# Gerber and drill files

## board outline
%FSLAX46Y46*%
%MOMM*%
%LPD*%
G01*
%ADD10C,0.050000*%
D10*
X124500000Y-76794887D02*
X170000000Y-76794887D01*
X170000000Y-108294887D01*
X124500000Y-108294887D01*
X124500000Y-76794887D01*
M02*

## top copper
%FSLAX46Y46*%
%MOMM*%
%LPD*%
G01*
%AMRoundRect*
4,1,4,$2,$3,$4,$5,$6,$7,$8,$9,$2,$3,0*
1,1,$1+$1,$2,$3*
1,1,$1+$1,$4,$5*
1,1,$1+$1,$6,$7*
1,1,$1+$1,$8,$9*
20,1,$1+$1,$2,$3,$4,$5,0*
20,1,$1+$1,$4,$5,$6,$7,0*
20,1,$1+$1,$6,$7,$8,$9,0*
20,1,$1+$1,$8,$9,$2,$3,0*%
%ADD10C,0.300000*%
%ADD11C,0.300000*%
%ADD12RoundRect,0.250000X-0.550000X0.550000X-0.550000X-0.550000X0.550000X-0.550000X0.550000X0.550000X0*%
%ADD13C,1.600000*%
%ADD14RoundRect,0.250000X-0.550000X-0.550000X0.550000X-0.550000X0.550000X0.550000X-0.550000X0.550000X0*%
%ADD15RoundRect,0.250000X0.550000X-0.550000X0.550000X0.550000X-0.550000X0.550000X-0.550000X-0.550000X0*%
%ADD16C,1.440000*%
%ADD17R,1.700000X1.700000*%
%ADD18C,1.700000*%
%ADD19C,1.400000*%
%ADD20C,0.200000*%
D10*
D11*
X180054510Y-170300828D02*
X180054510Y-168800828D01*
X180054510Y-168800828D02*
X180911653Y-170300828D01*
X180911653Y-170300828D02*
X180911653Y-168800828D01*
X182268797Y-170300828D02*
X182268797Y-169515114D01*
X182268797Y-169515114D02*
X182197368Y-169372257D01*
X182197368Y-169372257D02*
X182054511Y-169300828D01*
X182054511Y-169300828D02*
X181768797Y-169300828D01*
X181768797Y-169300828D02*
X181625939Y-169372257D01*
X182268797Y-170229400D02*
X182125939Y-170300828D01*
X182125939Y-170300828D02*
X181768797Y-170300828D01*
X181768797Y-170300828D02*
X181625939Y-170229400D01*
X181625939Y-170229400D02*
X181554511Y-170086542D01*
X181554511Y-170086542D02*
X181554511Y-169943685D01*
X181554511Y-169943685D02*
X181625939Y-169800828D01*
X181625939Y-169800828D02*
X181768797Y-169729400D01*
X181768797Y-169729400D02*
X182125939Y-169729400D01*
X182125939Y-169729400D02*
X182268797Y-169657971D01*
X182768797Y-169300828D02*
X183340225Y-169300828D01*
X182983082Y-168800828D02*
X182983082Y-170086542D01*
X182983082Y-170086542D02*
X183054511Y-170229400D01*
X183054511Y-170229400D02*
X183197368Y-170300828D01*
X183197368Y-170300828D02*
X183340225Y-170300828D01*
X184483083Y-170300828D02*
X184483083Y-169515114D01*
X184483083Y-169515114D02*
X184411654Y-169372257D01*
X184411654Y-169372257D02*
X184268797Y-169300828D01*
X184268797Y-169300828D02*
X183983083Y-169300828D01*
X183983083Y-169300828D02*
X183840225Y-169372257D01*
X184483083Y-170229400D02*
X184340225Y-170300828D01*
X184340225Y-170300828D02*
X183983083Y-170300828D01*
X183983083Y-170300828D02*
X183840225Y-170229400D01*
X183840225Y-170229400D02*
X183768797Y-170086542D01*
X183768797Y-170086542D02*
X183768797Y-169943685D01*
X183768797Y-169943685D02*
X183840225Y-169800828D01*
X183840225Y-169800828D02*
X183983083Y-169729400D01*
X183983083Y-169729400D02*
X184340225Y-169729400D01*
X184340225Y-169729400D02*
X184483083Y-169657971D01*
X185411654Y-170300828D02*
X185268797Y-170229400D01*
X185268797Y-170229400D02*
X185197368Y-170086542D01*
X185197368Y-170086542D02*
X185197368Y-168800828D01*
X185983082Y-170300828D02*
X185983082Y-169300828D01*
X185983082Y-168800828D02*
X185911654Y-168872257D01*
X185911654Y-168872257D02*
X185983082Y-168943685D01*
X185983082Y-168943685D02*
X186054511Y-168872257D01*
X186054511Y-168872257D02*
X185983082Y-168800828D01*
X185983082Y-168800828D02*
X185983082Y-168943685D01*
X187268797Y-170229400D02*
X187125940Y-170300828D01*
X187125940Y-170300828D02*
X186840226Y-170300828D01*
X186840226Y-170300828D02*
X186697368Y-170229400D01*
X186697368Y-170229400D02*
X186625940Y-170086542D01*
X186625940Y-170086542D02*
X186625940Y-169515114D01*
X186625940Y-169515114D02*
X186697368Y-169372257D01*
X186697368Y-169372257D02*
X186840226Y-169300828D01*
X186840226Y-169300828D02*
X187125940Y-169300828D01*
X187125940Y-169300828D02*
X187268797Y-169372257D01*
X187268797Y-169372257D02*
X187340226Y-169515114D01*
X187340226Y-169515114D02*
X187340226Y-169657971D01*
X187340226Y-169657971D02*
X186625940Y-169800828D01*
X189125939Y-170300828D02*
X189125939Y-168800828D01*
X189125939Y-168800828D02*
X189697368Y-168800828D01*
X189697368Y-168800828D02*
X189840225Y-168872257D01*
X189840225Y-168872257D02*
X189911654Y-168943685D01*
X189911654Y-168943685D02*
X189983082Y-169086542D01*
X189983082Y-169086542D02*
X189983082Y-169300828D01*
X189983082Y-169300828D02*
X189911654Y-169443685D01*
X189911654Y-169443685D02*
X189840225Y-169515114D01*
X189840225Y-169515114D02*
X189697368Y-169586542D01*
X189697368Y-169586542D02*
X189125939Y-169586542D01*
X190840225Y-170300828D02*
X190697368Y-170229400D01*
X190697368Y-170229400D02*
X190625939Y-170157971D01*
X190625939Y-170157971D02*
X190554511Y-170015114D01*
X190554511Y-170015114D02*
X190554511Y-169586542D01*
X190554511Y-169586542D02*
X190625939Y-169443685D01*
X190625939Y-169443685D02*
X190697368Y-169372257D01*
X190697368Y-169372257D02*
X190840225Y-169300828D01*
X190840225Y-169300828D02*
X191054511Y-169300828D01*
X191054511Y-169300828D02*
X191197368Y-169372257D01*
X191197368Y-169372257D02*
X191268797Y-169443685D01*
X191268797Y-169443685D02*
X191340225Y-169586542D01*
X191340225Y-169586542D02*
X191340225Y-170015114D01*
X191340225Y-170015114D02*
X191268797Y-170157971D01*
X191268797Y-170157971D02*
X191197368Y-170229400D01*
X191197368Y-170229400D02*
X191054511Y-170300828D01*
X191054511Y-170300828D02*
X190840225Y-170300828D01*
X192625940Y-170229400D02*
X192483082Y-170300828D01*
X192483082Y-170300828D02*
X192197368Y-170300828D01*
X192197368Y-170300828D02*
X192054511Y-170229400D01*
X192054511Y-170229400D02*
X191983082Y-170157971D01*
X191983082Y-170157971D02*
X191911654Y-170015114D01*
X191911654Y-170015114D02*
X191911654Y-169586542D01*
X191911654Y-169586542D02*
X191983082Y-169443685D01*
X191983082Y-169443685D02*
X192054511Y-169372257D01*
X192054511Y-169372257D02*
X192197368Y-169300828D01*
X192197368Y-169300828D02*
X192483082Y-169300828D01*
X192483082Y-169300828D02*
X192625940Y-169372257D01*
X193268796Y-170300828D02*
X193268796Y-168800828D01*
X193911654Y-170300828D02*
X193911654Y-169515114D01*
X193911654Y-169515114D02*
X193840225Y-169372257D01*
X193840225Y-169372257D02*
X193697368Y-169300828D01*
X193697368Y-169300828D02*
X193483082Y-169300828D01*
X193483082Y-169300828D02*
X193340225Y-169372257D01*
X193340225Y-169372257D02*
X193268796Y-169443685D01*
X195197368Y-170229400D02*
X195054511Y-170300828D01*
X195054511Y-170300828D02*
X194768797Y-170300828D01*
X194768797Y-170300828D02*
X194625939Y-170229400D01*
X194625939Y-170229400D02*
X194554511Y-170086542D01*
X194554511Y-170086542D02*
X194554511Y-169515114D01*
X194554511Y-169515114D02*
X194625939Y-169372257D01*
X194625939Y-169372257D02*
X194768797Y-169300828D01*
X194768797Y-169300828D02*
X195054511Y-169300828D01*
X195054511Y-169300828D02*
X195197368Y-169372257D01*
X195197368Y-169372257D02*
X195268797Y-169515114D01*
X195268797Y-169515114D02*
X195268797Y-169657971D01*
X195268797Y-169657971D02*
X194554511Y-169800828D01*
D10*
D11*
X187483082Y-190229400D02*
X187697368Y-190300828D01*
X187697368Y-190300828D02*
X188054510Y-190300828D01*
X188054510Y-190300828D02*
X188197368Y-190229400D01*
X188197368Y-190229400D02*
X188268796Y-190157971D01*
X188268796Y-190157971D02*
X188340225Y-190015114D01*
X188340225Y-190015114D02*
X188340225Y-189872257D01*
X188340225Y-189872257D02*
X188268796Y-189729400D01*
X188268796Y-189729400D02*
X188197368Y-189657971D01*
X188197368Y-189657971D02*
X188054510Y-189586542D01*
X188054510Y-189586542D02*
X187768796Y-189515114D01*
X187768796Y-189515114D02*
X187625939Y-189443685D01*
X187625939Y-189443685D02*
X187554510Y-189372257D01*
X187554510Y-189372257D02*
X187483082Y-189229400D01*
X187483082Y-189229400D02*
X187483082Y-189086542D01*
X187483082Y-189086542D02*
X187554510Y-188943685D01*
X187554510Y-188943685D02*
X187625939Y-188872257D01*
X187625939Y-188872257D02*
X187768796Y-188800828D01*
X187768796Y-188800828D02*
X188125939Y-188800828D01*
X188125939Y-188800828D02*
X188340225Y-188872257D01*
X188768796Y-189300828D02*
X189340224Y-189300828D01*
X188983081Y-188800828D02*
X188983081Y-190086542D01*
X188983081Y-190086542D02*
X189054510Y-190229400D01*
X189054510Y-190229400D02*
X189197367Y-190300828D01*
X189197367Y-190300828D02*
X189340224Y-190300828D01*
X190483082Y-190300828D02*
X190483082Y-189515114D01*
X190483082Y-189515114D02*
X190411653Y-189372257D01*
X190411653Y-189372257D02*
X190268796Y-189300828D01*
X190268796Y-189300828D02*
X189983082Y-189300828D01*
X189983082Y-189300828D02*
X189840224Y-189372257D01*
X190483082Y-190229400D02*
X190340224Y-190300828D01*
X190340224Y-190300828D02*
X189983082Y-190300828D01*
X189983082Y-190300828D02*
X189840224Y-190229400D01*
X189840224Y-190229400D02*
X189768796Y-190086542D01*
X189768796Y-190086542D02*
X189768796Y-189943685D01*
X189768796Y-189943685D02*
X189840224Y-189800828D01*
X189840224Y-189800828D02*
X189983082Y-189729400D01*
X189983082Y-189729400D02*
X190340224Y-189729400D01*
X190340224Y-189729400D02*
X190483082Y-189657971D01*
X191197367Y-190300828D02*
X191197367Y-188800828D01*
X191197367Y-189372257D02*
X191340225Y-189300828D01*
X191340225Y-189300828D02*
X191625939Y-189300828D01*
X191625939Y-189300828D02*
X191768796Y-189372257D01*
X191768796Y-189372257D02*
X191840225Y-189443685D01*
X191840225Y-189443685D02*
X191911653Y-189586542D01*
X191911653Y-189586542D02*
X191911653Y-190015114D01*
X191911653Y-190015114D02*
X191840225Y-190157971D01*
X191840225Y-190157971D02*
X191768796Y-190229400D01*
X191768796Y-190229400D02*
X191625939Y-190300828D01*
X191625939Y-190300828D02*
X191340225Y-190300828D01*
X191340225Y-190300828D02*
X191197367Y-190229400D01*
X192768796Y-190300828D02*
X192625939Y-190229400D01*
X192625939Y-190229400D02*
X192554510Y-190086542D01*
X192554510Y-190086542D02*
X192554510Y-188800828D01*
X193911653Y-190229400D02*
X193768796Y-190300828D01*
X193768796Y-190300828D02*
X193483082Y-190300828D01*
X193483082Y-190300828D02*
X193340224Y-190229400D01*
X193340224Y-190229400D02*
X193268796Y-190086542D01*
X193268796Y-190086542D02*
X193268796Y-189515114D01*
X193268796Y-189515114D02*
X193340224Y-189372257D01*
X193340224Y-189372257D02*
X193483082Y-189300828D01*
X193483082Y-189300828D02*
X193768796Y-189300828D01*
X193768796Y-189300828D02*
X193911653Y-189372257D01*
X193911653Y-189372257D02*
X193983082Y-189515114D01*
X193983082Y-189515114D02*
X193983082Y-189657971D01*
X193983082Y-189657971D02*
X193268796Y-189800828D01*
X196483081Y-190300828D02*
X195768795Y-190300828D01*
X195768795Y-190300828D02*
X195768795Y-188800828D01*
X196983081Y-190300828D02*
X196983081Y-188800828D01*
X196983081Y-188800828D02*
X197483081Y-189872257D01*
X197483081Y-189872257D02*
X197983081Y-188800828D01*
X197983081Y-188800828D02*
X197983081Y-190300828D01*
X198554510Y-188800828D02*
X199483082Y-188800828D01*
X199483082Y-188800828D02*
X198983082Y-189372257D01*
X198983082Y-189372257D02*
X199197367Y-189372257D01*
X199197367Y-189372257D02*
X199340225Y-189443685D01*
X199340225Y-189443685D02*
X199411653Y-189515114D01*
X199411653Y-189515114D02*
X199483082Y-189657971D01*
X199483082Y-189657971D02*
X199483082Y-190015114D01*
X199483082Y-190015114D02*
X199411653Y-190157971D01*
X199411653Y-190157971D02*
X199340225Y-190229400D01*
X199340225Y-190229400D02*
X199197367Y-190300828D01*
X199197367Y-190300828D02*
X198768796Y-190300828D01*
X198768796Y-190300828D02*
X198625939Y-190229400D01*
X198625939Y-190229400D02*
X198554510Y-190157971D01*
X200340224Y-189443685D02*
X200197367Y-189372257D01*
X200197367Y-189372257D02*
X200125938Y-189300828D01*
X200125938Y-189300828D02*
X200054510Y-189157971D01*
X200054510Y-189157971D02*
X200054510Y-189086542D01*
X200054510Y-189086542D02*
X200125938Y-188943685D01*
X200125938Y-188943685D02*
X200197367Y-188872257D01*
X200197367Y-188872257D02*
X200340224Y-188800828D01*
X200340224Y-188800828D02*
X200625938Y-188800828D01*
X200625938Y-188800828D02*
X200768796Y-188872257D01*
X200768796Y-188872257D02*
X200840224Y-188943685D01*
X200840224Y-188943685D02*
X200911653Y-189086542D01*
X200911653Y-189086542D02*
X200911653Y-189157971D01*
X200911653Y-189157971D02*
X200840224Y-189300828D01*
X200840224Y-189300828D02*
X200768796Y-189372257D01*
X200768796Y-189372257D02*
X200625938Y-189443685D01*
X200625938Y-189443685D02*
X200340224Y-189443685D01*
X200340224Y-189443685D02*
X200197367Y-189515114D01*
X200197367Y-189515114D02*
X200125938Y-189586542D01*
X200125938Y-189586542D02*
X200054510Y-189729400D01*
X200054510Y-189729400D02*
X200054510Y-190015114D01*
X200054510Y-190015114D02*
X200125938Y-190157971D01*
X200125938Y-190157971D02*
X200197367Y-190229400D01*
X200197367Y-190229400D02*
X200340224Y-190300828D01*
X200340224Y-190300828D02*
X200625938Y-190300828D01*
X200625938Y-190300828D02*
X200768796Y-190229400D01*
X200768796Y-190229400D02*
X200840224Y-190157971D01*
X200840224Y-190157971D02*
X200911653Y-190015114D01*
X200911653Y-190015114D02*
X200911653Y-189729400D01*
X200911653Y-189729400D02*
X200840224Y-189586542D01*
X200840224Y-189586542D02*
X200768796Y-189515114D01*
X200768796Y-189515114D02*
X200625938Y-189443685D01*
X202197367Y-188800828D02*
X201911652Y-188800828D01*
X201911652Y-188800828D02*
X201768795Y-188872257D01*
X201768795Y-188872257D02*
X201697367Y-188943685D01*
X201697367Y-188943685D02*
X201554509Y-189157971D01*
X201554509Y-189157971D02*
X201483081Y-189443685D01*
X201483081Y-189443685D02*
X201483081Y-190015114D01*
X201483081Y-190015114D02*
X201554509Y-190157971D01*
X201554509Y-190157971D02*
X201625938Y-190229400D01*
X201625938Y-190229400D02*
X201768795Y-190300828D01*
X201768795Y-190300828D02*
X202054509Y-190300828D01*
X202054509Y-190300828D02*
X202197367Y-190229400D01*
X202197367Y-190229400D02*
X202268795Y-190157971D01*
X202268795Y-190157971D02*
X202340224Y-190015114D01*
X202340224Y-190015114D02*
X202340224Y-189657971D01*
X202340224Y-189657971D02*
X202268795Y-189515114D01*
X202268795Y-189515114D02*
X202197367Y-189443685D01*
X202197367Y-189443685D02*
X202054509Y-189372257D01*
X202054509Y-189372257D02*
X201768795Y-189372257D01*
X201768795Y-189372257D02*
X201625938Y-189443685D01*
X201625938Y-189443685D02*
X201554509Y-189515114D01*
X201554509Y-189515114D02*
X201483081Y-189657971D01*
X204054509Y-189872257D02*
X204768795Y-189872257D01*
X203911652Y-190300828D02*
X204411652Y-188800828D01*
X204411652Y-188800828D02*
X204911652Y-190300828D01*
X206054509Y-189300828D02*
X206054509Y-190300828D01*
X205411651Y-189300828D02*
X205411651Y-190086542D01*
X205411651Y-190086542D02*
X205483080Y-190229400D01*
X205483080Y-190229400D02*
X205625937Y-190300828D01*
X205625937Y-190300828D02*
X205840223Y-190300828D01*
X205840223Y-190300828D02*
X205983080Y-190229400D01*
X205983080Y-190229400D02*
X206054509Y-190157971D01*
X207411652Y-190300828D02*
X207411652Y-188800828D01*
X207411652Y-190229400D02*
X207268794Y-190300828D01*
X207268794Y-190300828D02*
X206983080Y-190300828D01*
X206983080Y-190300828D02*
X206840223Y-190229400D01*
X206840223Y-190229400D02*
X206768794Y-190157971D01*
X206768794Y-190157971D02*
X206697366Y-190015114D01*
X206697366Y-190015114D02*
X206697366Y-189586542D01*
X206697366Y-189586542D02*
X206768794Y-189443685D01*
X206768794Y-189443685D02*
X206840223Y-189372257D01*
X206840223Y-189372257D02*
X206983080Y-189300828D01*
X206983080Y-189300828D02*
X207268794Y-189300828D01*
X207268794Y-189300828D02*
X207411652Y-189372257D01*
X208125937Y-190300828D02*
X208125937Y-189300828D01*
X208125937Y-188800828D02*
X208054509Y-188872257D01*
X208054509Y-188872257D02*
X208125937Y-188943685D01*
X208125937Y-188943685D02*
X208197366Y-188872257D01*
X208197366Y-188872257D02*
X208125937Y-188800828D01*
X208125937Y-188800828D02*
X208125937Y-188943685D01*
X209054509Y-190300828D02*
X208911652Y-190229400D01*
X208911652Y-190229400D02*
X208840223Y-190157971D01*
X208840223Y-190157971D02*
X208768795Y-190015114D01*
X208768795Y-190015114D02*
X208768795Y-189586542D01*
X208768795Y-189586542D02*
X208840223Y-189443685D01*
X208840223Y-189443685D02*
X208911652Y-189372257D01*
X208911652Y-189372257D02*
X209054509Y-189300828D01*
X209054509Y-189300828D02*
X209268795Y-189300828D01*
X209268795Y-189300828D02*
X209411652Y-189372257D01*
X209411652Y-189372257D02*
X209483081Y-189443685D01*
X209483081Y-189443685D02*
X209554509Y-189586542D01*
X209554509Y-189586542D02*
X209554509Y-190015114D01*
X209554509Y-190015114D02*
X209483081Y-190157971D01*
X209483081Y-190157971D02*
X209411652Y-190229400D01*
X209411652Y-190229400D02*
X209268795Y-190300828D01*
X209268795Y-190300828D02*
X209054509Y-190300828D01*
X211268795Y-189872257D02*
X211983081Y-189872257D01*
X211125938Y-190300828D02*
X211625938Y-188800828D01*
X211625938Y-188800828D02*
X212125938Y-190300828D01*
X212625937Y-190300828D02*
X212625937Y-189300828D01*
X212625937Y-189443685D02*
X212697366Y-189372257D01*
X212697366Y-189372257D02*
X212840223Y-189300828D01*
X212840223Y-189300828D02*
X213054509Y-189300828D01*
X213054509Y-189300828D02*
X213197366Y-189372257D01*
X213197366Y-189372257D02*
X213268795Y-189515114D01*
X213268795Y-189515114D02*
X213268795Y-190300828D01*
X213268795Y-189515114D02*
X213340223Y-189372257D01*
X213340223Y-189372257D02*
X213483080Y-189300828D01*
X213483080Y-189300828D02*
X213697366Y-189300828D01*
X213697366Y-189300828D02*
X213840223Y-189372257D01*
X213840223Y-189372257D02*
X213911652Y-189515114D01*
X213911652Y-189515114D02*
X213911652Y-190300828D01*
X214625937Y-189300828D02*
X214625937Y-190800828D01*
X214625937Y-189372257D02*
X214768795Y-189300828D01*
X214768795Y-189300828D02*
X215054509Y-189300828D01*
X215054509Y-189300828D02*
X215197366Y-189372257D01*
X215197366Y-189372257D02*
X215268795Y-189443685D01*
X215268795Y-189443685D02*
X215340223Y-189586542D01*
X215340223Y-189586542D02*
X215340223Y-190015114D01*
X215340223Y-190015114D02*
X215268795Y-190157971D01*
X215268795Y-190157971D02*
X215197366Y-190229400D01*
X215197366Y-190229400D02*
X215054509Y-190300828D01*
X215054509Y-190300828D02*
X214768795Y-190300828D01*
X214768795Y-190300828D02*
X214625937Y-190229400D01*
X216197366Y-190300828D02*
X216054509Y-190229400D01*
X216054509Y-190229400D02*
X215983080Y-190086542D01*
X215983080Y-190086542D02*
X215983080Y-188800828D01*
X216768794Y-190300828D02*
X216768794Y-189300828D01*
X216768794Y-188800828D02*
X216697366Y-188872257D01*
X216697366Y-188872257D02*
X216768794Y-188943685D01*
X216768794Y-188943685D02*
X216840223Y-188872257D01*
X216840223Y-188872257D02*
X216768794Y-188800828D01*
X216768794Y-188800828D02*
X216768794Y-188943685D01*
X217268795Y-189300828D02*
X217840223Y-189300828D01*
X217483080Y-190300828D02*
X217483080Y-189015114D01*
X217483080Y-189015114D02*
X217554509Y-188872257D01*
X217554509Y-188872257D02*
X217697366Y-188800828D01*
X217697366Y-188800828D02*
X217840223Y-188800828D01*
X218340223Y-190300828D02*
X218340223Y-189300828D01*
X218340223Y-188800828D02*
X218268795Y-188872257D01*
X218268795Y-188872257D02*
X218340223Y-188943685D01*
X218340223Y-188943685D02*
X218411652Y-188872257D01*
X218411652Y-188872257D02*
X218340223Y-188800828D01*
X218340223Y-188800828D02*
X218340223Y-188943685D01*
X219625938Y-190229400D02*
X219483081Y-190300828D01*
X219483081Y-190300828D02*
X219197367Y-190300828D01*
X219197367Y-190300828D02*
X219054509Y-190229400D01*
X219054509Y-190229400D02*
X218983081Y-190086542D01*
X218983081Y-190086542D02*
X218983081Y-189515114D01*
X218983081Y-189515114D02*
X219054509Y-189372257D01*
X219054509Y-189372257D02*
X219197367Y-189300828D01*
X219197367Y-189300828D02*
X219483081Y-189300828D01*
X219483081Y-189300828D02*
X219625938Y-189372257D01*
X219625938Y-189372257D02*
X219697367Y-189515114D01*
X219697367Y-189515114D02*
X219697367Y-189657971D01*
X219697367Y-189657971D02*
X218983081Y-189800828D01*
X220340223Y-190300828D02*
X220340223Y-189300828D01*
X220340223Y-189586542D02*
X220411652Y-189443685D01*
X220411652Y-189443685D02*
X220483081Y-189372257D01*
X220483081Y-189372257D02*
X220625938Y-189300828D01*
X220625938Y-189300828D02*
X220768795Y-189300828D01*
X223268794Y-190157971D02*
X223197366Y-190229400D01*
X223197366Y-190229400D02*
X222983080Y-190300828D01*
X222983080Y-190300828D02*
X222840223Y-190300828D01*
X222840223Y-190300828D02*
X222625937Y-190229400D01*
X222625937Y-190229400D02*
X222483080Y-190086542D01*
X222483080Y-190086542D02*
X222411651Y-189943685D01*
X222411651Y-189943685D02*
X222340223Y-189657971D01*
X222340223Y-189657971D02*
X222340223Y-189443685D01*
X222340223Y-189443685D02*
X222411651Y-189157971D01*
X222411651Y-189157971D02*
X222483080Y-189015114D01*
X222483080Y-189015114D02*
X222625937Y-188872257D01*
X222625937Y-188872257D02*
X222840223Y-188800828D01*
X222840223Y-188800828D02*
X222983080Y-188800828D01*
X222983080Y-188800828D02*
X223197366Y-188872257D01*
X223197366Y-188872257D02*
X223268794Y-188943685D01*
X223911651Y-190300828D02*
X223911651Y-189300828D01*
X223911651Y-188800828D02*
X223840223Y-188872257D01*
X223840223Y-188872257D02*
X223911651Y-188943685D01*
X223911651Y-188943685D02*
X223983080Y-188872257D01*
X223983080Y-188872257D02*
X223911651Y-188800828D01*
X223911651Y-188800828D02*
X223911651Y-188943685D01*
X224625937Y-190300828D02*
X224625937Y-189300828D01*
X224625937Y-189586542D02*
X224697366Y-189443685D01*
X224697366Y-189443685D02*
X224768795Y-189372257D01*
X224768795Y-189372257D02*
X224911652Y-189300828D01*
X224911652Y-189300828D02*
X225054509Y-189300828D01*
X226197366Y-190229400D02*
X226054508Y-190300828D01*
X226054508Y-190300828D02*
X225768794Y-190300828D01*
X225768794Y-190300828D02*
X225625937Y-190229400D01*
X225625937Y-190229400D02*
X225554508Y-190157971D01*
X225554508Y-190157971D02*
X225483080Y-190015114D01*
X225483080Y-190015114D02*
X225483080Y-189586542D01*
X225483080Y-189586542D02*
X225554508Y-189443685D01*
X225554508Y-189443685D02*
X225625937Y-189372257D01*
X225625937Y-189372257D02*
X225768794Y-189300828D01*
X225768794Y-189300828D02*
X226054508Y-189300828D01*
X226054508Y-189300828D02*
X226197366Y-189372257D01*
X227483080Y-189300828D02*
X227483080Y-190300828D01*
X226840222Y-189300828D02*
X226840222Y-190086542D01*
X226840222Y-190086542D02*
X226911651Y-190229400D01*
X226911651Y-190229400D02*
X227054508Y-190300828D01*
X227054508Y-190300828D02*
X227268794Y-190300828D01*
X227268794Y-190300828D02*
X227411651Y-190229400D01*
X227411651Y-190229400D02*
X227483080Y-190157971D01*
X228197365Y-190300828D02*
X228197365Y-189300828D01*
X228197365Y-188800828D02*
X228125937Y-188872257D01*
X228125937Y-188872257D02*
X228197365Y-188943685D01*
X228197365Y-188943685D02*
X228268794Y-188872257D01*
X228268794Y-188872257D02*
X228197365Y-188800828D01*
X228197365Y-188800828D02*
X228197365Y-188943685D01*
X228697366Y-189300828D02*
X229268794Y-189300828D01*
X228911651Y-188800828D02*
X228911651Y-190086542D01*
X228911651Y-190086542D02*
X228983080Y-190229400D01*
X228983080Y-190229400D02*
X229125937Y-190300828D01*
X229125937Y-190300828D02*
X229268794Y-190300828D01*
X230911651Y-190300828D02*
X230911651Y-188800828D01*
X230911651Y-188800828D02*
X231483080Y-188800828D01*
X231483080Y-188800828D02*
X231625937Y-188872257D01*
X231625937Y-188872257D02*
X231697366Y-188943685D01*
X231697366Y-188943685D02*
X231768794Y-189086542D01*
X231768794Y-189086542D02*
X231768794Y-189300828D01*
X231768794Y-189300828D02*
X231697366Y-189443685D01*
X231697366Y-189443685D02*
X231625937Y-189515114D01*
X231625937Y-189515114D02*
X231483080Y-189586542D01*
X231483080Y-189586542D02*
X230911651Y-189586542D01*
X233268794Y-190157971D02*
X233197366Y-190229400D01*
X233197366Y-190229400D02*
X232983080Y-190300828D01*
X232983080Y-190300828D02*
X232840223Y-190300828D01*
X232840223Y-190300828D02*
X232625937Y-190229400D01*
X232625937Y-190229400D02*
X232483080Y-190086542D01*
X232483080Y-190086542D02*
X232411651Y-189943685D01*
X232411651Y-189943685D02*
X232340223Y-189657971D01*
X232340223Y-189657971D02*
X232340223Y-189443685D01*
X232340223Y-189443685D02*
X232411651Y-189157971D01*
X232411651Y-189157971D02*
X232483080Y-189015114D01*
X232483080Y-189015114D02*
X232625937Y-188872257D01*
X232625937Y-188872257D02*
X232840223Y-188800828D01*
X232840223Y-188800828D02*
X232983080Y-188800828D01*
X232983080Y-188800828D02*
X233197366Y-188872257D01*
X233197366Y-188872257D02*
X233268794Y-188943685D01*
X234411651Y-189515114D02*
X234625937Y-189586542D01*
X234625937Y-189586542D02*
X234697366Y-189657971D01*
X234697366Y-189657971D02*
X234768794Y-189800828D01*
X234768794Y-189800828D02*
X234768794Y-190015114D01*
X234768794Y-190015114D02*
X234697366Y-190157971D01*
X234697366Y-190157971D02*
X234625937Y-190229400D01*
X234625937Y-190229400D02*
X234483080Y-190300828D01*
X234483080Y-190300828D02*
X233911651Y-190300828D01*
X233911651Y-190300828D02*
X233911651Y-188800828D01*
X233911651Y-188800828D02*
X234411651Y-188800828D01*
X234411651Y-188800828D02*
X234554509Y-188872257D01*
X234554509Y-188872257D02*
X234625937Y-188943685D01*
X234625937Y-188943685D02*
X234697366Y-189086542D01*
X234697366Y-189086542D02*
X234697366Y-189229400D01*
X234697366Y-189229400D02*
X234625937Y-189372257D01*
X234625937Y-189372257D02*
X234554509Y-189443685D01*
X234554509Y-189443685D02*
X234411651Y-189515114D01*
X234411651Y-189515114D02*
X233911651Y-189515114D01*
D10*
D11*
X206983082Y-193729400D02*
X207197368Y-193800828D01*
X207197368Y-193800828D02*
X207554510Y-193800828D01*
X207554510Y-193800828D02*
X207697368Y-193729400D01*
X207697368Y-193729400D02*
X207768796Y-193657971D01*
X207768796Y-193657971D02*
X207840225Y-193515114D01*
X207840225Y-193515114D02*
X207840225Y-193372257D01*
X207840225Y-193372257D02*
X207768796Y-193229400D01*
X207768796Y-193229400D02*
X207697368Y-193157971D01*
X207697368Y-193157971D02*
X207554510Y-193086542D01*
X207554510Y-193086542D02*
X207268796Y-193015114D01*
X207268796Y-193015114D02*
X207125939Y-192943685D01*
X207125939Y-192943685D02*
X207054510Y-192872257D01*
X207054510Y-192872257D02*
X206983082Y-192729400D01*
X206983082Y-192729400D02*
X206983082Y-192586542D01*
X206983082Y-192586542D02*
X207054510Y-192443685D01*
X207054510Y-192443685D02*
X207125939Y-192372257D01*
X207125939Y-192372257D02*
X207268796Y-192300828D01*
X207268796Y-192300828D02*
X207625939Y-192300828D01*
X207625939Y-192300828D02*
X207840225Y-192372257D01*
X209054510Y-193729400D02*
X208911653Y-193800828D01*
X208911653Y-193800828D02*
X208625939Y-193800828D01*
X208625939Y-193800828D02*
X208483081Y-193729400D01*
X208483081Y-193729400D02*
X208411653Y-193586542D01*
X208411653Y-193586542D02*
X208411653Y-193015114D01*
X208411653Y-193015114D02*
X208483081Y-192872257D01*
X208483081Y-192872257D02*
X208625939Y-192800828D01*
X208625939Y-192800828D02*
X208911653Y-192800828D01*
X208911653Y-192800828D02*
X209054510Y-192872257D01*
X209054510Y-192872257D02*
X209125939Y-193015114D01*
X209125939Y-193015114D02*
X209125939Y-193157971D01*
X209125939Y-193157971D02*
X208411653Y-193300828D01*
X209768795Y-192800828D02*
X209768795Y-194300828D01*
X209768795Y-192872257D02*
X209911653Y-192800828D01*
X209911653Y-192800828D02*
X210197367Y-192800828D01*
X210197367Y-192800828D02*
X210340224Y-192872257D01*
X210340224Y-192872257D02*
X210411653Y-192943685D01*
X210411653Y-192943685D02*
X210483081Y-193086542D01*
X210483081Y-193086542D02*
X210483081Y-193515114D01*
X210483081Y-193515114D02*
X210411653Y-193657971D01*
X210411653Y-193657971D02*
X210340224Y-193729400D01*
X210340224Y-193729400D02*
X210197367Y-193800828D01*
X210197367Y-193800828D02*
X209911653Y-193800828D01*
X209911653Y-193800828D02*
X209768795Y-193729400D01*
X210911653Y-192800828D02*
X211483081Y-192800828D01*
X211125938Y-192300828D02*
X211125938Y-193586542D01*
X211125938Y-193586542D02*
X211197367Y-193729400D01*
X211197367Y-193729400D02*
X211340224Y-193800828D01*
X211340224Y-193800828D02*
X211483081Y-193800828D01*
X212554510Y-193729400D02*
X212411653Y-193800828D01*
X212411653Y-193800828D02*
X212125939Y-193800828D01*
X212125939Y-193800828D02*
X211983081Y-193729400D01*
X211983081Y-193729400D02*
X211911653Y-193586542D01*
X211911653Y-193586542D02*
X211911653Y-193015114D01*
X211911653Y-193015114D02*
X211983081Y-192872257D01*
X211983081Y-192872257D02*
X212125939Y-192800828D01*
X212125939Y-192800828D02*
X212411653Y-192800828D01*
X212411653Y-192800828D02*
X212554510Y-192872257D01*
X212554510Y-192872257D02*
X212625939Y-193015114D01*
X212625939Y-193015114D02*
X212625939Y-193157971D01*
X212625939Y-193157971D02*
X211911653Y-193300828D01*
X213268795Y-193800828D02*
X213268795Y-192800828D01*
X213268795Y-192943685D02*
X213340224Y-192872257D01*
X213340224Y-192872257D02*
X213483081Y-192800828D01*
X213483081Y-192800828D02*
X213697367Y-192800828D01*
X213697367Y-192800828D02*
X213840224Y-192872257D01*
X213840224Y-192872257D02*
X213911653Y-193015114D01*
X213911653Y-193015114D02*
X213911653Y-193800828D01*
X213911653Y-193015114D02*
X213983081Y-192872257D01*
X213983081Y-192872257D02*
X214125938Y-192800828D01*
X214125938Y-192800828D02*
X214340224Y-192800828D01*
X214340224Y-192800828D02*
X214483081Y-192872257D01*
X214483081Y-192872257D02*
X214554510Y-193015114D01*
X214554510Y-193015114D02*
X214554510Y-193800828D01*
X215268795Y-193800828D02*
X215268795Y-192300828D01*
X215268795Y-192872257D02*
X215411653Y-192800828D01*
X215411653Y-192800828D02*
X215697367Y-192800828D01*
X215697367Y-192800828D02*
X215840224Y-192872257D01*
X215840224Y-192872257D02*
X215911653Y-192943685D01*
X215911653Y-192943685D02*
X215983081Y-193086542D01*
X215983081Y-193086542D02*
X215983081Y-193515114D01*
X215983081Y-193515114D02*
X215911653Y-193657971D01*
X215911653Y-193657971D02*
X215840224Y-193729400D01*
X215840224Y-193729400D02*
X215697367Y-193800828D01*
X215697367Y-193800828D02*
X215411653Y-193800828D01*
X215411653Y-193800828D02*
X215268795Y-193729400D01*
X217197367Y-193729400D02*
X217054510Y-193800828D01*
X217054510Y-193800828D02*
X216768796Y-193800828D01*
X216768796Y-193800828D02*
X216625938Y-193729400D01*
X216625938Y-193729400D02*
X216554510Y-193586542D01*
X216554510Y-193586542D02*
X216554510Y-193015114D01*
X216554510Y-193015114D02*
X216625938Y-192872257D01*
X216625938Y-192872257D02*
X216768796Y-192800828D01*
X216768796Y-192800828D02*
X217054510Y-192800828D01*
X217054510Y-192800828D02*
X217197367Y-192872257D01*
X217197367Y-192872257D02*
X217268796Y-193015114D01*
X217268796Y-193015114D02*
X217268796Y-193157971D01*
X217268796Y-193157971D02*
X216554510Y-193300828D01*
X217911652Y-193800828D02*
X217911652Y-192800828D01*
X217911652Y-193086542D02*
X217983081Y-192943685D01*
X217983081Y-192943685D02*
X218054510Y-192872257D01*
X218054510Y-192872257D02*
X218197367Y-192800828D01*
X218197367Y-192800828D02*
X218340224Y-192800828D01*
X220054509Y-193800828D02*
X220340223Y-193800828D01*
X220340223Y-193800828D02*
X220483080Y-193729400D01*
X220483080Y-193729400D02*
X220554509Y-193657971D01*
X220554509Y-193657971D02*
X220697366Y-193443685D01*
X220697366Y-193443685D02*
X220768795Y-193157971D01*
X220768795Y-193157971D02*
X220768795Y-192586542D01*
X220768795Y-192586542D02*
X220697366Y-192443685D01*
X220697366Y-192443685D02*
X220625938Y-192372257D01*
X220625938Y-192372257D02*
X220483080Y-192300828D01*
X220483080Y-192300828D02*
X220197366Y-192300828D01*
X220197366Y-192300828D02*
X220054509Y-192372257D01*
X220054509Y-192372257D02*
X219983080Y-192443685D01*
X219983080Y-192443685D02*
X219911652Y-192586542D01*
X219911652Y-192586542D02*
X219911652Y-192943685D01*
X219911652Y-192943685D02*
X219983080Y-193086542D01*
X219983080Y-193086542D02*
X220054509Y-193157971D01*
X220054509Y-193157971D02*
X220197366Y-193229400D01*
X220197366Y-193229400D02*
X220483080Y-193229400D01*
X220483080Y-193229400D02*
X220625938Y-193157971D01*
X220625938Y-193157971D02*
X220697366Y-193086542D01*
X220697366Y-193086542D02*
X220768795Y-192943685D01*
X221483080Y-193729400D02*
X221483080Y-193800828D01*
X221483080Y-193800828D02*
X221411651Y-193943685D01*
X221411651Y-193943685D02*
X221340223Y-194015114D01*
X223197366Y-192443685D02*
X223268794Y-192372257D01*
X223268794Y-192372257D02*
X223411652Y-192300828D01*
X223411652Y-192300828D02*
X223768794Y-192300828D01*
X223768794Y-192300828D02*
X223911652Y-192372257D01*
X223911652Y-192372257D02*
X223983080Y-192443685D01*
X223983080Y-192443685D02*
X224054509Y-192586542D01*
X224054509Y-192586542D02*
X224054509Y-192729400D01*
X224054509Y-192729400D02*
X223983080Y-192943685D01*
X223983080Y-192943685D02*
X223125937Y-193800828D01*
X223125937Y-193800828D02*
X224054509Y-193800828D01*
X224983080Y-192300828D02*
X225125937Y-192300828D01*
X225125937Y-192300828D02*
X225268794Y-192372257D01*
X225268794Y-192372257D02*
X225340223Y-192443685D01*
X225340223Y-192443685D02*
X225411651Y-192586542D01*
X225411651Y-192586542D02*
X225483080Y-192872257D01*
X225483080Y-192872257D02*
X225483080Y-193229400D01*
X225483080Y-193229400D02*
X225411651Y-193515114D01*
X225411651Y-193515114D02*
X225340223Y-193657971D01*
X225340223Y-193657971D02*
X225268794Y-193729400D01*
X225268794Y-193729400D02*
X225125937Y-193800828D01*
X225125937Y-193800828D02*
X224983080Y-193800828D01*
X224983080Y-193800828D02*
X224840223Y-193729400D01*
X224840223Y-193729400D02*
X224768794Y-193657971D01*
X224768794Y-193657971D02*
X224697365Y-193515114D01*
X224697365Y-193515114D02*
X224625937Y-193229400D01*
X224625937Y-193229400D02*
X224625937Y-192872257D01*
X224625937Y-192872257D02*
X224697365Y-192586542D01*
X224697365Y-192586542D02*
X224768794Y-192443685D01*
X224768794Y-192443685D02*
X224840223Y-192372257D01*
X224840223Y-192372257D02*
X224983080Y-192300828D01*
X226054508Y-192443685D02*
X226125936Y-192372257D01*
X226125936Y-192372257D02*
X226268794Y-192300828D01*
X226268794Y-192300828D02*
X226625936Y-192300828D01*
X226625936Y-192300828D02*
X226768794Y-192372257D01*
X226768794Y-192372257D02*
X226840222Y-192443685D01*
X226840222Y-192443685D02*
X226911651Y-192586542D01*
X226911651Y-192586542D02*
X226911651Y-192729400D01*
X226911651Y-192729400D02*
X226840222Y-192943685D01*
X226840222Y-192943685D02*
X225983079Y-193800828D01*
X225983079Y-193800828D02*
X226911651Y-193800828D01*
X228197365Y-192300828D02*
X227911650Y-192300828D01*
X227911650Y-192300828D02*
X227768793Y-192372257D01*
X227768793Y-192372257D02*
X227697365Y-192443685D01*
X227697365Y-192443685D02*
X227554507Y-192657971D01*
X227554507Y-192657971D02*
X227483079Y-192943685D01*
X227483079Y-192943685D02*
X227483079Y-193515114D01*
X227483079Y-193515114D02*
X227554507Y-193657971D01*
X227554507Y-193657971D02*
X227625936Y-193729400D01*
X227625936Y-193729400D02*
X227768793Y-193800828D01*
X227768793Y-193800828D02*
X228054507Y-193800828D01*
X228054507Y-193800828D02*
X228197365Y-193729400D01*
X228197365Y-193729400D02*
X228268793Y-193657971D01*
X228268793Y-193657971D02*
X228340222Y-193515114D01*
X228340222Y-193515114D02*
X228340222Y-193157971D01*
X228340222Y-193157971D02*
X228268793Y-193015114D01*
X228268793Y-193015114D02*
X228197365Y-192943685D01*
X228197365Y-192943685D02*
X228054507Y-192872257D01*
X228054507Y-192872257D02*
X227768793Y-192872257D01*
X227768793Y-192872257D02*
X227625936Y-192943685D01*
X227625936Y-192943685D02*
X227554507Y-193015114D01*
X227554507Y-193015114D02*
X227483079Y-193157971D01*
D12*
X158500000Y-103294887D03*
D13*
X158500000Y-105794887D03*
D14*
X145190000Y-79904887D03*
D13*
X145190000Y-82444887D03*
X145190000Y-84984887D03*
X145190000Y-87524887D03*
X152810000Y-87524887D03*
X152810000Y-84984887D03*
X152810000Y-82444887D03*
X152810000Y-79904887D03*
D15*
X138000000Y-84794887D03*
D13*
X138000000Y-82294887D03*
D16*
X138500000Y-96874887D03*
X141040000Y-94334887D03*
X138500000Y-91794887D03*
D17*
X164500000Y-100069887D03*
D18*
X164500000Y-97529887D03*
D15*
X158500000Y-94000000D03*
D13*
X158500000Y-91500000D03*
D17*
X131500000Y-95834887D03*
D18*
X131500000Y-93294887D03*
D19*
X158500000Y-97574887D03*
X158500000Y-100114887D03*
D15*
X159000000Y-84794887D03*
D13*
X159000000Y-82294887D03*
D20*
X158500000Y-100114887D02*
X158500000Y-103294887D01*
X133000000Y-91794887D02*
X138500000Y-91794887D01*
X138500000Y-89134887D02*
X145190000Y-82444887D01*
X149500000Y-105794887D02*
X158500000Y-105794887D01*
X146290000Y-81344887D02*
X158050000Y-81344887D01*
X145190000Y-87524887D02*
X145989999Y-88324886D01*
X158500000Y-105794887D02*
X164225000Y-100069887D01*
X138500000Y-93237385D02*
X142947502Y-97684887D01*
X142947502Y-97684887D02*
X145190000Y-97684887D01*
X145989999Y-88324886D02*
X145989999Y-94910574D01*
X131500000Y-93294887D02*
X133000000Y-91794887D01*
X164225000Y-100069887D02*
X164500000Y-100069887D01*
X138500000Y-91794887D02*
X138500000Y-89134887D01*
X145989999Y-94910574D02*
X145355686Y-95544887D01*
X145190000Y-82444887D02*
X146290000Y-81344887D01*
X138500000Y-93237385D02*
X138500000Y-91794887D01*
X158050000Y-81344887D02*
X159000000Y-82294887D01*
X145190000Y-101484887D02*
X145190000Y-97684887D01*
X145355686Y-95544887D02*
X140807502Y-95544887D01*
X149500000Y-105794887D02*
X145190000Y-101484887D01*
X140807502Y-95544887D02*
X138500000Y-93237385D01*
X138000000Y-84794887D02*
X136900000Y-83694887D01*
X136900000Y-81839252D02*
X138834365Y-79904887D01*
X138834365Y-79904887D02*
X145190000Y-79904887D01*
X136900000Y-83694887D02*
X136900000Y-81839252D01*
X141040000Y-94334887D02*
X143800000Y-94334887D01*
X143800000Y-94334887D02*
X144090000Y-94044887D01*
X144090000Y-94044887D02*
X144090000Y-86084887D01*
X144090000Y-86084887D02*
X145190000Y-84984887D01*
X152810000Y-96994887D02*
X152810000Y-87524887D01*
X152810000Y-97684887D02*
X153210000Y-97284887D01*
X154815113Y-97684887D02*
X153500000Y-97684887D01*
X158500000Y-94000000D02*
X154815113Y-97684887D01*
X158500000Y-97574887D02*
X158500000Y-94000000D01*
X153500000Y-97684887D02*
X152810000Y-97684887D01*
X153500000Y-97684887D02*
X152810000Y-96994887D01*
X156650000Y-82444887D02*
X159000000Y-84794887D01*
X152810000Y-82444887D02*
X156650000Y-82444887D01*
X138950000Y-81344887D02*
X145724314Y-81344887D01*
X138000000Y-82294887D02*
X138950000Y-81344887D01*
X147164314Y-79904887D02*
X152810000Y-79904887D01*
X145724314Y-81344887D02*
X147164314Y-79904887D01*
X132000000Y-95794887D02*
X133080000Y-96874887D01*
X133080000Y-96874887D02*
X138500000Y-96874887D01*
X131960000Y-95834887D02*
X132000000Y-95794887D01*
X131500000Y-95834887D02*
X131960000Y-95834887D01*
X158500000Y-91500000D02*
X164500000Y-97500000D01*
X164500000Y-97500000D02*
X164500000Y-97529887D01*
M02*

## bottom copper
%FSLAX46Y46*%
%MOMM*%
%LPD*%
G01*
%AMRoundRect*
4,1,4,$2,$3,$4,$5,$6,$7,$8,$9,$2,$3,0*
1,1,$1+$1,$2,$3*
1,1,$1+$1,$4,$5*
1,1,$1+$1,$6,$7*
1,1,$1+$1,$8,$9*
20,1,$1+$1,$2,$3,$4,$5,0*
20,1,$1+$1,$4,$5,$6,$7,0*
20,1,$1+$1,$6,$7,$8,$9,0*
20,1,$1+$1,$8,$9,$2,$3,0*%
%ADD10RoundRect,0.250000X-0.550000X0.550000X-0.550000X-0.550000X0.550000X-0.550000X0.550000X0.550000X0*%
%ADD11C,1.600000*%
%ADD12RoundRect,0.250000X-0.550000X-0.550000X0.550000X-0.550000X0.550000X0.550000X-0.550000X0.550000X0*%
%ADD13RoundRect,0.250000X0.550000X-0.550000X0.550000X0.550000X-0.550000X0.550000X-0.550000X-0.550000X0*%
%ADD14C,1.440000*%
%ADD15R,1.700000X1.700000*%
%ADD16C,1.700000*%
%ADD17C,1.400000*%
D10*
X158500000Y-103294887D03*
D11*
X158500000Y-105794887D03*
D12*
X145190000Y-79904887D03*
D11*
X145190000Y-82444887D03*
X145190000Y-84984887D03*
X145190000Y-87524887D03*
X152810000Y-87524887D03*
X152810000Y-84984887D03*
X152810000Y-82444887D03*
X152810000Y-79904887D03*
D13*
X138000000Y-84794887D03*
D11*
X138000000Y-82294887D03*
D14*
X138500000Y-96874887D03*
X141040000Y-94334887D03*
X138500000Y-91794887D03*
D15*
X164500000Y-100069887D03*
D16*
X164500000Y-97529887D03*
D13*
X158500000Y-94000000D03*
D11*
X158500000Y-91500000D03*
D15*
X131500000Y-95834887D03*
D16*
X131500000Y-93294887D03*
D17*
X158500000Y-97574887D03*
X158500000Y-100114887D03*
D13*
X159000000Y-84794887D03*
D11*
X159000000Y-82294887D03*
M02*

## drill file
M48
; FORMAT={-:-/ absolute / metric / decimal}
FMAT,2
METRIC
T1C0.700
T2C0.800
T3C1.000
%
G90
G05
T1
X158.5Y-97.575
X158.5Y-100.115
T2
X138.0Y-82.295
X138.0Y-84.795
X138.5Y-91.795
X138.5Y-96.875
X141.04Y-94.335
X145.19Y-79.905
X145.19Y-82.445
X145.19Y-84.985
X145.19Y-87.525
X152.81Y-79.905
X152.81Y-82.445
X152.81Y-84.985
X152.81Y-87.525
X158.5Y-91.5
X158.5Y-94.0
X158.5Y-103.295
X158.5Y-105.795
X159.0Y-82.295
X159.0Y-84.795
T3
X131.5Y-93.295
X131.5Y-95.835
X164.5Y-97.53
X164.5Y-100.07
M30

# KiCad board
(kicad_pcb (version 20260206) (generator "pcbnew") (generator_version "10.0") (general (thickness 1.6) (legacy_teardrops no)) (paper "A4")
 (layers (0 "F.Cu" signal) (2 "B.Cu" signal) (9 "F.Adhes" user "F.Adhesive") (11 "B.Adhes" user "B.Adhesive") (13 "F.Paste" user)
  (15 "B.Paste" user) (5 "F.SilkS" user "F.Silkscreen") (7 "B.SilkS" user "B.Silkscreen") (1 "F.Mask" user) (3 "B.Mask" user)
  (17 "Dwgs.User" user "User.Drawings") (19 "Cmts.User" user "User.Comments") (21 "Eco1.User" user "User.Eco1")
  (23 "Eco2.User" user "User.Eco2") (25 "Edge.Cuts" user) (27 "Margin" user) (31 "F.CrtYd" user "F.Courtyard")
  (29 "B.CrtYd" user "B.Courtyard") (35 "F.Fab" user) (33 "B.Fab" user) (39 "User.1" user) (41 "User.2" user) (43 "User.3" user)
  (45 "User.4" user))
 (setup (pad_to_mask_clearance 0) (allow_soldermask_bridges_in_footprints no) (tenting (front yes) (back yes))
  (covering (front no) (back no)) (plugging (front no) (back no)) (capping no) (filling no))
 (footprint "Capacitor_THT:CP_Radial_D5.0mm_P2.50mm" (layer "F.Cu") (at 158.5 103.294887 -90)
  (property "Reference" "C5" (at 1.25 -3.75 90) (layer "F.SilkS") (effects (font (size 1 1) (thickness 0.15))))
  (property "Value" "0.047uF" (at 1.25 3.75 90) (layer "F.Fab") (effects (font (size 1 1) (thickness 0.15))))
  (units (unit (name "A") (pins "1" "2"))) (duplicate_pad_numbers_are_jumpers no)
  (pad "1" thru_hole roundrect (at 0 0 270) (size 1.6 1.6) (drill 0.8) (layers "*.Cu" "*.Mask") (remove_unused_layers no)
   (roundrect_rratio 0.15625) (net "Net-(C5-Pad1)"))
  (pad "2" thru_hole circle (at 2.5 0 270) (size 1.6 1.6) (drill 0.8) (layers "*.Cu" "*.Mask") (remove_unused_layers no) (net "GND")))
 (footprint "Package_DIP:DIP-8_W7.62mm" (layer "F.Cu") (at 145.19 79.904887)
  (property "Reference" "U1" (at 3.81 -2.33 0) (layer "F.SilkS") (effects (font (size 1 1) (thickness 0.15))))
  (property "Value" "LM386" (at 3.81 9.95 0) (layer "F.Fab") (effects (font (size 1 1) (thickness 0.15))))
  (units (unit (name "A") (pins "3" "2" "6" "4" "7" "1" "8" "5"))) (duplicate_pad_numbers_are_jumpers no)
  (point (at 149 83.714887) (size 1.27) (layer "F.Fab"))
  (pad "1" thru_hole roundrect (at 0 0) (size 1.6 1.6) (drill 0.8) (layers "*.Cu" "*.Mask") (remove_unused_layers no)
   (roundrect_rratio 0.15625) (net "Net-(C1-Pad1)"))
  (pad "2" thru_hole circle (at 0 2.54) (size 1.6 1.6) (drill 0.8) (layers "*.Cu" "*.Mask") (remove_unused_layers no) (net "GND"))
  (pad "3" thru_hole circle (at 0 5.08) (size 1.6 1.6) (drill 0.8) (layers "*.Cu" "*.Mask") (remove_unused_layers no) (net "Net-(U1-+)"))
  (pad "4" thru_hole circle (at 0 7.62) (size 1.6 1.6) (drill 0.8) (layers "*.Cu" "*.Mask") (remove_unused_layers no) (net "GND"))
  (pad "5" thru_hole circle (at 7.62 7.62) (size 1.6 1.6) (drill 0.8) (layers "*.Cu" "*.Mask") (remove_unused_layers no)
   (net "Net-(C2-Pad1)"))
  (pad "6" thru_hole circle (at 7.62 5.08) (size 1.6 1.6) (drill 0.8) (layers "*.Cu" "*.Mask") (remove_unused_layers no) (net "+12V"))
  (pad "7" thru_hole circle (at 7.62 2.54) (size 1.6 1.6) (drill 0.8) (layers "*.Cu" "*.Mask") (remove_unused_layers no)
   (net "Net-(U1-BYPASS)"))
  (pad "8" thru_hole circle (at 7.62 0) (size 1.6 1.6) (drill 0.8) (layers "*.Cu" "*.Mask") (remove_unused_layers no) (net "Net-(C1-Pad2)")))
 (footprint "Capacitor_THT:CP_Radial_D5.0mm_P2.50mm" (layer "F.Cu") (at 138 84.794887 90)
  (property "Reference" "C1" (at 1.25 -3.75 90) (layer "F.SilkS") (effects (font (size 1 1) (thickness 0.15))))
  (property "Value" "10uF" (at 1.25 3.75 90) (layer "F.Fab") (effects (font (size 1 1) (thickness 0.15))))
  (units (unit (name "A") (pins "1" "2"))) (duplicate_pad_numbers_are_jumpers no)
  (pad "1" thru_hole roundrect (at 0 0 90) (size 1.6 1.6) (drill 0.8) (layers "*.Cu" "*.Mask") (remove_unused_layers no)
   (roundrect_rratio 0.15625) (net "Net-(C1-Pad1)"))
  (pad "2" thru_hole circle (at 2.5 0 90) (size 1.6 1.6) (drill 0.8) (layers "*.Cu" "*.Mask") (remove_unused_layers no)
   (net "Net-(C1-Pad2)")))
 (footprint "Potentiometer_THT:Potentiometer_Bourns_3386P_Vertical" (layer "F.Cu") (at 138.5 96.874887)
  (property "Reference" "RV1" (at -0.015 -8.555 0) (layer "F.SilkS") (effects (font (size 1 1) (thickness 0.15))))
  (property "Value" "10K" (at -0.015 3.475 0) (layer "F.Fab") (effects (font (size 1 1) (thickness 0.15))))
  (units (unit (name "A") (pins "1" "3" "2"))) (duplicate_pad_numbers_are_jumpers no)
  (pad "1" thru_hole circle (at 0 0) (size 1.44 1.44) (drill 0.8) (layers "*.Cu" "*.Mask") (remove_unused_layers no) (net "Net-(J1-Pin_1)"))
  (pad "2" thru_hole circle (at 2.54 -2.54) (size 1.44 1.44) (drill 0.8) (layers "*.Cu" "*.Mask") (remove_unused_layers no)
   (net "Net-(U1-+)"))
  (pad "3" thru_hole circle (at 0 -5.08) (size 1.44 1.44) (drill 0.8) (layers "*.Cu" "*.Mask") (remove_unused_layers no) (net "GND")))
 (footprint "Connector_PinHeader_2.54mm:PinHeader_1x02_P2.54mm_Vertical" (layer "F.Cu") (at 164.5 100.069887 180)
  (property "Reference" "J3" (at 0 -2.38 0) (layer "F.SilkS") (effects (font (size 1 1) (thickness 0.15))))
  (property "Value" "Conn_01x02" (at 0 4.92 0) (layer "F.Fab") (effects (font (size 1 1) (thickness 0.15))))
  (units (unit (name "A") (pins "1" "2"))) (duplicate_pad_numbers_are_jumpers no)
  (pad "1" thru_hole rect (at 0 0 180) (size 1.7 1.7) (drill 1) (layers "*.Cu" "*.Mask") (remove_unused_layers no) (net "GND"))
  (pad "2" thru_hole circle (at 0 2.54 180) (size 1.7 1.7) (drill 1) (layers "*.Cu" "*.Mask") (remove_unused_layers no)
   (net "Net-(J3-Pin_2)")))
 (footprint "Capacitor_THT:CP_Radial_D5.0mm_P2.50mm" (layer "F.Cu") (at 158.5 94 90)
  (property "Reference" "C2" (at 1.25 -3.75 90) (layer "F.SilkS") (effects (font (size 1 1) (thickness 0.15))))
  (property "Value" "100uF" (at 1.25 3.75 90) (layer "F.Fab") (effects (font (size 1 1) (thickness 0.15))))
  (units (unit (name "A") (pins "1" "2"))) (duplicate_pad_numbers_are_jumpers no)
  (pad "1" thru_hole roundrect (at 0 0 90) (size 1.6 1.6) (drill 0.8) (layers "*.Cu" "*.Mask") (remove_unused_layers no)
   (roundrect_rratio 0.15625) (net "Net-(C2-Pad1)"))
  (pad "2" thru_hole circle (at 2.5 0 90) (size 1.6 1.6) (drill 0.8) (layers "*.Cu" "*.Mask") (remove_unused_layers no)
   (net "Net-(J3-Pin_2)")))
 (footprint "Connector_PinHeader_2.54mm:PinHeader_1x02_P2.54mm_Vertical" (layer "F.Cu") (at 131.5 95.834887 180)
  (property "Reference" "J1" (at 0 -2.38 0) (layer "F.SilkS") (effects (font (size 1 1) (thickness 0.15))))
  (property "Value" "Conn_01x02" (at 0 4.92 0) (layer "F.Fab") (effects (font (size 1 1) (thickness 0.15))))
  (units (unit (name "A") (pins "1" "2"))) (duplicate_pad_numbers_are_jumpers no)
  (pad "1" thru_hole rect (at 0 0 180) (size 1.7 1.7) (drill 1) (layers "*.Cu" "*.Mask") (remove_unused_layers no) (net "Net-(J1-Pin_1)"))
  (pad "2" thru_hole circle (at 0 2.54 180) (size 1.7 1.7) (drill 1) (layers "*.Cu" "*.Mask") (remove_unused_layers no) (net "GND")))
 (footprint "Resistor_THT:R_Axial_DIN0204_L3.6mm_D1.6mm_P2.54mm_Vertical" (layer "F.Cu") (at 158.5 97.574887 -90)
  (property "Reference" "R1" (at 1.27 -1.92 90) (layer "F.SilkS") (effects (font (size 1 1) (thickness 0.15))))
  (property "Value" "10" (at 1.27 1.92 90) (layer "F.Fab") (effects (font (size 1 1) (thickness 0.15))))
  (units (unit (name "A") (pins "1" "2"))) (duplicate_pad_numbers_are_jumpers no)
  (pad "1" thru_hole circle (at 0 0 270) (size 1.4 1.4) (drill 0.7) (layers "*.Cu" "*.Mask") (remove_unused_layers no) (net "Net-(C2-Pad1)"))
  (pad "2" thru_hole circle (at 2.54 0 270) (size 1.4 1.4) (drill 0.7) (layers "*.Cu" "*.Mask") (remove_unused_layers no)
   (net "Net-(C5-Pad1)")))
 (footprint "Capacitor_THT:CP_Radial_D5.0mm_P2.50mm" (layer "F.Cu") (at 159 84.794887 90)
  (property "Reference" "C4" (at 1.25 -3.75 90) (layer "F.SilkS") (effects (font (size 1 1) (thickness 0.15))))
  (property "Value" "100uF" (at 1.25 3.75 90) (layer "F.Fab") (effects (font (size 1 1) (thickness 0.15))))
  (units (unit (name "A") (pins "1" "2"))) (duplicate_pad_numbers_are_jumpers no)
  (pad "1" thru_hole roundrect (at 0 0 90) (size 1.6 1.6) (drill 0.8) (layers "*.Cu" "*.Mask") (remove_unused_layers no)
   (roundrect_rratio 0.15625) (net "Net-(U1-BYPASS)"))
  (pad "2" thru_hole circle (at 2.5 0 90) (size 1.6 1.6) (drill 0.8) (layers "*.Cu" "*.Mask") (remove_unused_layers no) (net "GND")))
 (gr_rect (start 124.5 76.794887) (end 170 108.294887) (stroke (width 0.05) (type solid)) (fill no) (layer "Edge.Cuts"))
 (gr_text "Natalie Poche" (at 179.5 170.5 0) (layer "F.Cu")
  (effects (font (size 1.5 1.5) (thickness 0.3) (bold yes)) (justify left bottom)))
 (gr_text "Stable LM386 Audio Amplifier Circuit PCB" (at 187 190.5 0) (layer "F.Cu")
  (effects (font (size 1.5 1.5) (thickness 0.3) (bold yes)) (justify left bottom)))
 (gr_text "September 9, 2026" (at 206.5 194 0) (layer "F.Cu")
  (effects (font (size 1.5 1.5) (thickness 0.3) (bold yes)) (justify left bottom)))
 (segment (start 158.5 100.114887) (end 158.5 103.294887) (width 0.2) (layer "F.Cu") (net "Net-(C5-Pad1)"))
 (segment (start 133 91.794887) (end 138.5 91.794887) (width 0.2) (layer "F.Cu") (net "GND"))
 (segment (start 138.5 89.134887) (end 145.19 82.444887) (width 0.2) (layer "F.Cu") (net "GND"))
 (segment (start 149.5 105.794887) (end 158.5 105.794887) (width 0.2) (layer "F.Cu") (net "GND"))
 (segment (start 146.29 81.344887) (end 158.05 81.344887) (width 0.2) (layer "F.Cu") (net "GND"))
 (segment (start 145.19 87.524887) (end 145.989999 88.324886) (width 0.2) (layer "F.Cu") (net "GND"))
 (segment (start 158.5 105.794887) (end 164.225 100.069887) (width 0.2) (layer "F.Cu") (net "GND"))
 (segment (start 138.5 93.237385) (end 142.947502 97.684887) (width 0.2) (layer "F.Cu") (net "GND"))
 (segment (start 142.947502 97.684887) (end 145.19 97.684887) (width 0.2) (layer "F.Cu") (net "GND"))
 (segment (start 145.989999 88.324886) (end 145.989999 94.910574) (width 0.2) (layer "F.Cu") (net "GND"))
 (segment (start 131.5 93.294887) (end 133 91.794887) (width 0.2) (layer "F.Cu") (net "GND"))
 (segment (start 164.225 100.069887) (end 164.5 100.069887) (width 0.2) (layer "F.Cu") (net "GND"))
 (segment (start 138.5 91.794887) (end 138.5 89.134887) (width 0.2) (layer "F.Cu") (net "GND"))
 (segment (start 145.989999 94.910574) (end 145.355686 95.544887) (width 0.2) (layer "F.Cu") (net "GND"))
 (segment (start 145.19 82.444887) (end 146.29 81.344887) (width 0.2) (layer "F.Cu") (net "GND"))
 (segment (start 138.5 93.237385) (end 138.5 91.794887) (width 0.2) (layer "F.Cu") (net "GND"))
 (segment (start 158.05 81.344887) (end 159 82.294887) (width 0.2) (layer "F.Cu") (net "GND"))
 (segment (start 145.19 101.484887) (end 145.19 97.684887) (width 0.2) (layer "F.Cu") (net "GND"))
 (segment (start 145.355686 95.544887) (end 140.807502 95.544887) (width 0.2) (layer "F.Cu") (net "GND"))
 (segment (start 149.5 105.794887) (end 145.19 101.484887) (width 0.2) (layer "F.Cu") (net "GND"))
 (segment (start 140.807502 95.544887) (end 138.5 93.237385) (width 0.2) (layer "F.Cu") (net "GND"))
 (segment (start 138 84.794887) (end 136.9 83.694887) (width 0.2) (layer "F.Cu") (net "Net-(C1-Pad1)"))
 (segment (start 136.9 81.839252) (end 138.834365 79.904887) (width 0.2) (layer "F.Cu") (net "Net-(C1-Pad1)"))
 (segment (start 138.834365 79.904887) (end 145.19 79.904887) (width 0.2) (layer "F.Cu") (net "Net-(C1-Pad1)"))
 (segment (start 136.9 83.694887) (end 136.9 81.839252) (width 0.2) (layer "F.Cu") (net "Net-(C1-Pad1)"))
 (segment (start 141.04 94.334887) (end 143.8 94.334887) (width 0.2) (layer "F.Cu") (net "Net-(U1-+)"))
 (segment (start 143.8 94.334887) (end 144.09 94.044887) (width 0.2) (layer "F.Cu") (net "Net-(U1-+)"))
 (segment (start 144.09 94.044887) (end 144.09 86.084887) (width 0.2) (layer "F.Cu") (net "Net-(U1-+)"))
 (segment (start 144.09 86.084887) (end 145.19 84.984887) (width 0.2) (layer "F.Cu") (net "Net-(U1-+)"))
 (segment (start 152.81 96.994887) (end 152.81 87.524887) (width 0.2) (layer "F.Cu") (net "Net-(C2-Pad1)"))
 (segment (start 152.81 97.684887) (end 153.21 97.284887) (width 0.2) (layer "F.Cu") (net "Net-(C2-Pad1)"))
 (segment (start 154.815113 97.684887) (end 153.5 97.684887) (width 0.2) (layer "F.Cu") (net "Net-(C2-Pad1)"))
 (segment (start 158.5 94) (end 154.815113 97.684887) (width 0.2) (layer "F.Cu") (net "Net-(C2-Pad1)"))
 (segment (start 158.5 97.574887) (end 158.5 94) (width 0.2) (layer "F.Cu") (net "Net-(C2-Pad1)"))
 (segment (start 153.5 97.684887) (end 152.81 97.684887) (width 0.2) (layer "F.Cu") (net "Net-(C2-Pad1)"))
 (segment (start 153.5 97.684887) (end 152.81 96.994887) (width 0.2) (layer "F.Cu") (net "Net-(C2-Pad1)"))
 (segment (start 156.65 82.444887) (end 159 84.794887) (width 0.2) (layer "F.Cu") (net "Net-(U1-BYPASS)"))
 (segment (start 152.81 82.444887) (end 156.65 82.444887) (width 0.2) (layer "F.Cu") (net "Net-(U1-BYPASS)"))
 (segment (start 138.95 81.344887) (end 145.724314 81.344887) (width 0.2) (layer "F.Cu") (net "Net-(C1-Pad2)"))
 (segment (start 138 82.294887) (end 138.95 81.344887) (width 0.2) (layer "F.Cu") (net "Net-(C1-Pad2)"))
 (segment (start 147.164314 79.904887) (end 152.81 79.904887) (width 0.2) (layer "F.Cu") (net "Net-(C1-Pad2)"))
 (segment (start 145.724314 81.344887) (end 147.164314 79.904887) (width 0.2) (layer "F.Cu") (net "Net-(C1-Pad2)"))
 (segment (start 132 95.794887) (end 133.08 96.874887) (width 0.2) (layer "F.Cu") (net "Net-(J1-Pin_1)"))
 (segment (start 133.08 96.874887) (end 138.5 96.874887) (width 0.2) (layer "F.Cu") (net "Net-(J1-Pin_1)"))
 (segment (start 131.96 95.834887) (end 132 95.794887) (width 0.2) (layer "F.Cu") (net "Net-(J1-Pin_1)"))
 (segment (start 131.5 95.834887) (end 131.96 95.834887) (width 0.2) (layer "F.Cu") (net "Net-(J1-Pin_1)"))
 (segment (start 158.5 91.5) (end 164.5 97.5) (width 0.2) (layer "F.Cu") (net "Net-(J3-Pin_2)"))
 (segment (start 164.5 97.5) (end 164.5 97.529887) (width 0.2) (layer "F.Cu") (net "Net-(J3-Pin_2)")))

